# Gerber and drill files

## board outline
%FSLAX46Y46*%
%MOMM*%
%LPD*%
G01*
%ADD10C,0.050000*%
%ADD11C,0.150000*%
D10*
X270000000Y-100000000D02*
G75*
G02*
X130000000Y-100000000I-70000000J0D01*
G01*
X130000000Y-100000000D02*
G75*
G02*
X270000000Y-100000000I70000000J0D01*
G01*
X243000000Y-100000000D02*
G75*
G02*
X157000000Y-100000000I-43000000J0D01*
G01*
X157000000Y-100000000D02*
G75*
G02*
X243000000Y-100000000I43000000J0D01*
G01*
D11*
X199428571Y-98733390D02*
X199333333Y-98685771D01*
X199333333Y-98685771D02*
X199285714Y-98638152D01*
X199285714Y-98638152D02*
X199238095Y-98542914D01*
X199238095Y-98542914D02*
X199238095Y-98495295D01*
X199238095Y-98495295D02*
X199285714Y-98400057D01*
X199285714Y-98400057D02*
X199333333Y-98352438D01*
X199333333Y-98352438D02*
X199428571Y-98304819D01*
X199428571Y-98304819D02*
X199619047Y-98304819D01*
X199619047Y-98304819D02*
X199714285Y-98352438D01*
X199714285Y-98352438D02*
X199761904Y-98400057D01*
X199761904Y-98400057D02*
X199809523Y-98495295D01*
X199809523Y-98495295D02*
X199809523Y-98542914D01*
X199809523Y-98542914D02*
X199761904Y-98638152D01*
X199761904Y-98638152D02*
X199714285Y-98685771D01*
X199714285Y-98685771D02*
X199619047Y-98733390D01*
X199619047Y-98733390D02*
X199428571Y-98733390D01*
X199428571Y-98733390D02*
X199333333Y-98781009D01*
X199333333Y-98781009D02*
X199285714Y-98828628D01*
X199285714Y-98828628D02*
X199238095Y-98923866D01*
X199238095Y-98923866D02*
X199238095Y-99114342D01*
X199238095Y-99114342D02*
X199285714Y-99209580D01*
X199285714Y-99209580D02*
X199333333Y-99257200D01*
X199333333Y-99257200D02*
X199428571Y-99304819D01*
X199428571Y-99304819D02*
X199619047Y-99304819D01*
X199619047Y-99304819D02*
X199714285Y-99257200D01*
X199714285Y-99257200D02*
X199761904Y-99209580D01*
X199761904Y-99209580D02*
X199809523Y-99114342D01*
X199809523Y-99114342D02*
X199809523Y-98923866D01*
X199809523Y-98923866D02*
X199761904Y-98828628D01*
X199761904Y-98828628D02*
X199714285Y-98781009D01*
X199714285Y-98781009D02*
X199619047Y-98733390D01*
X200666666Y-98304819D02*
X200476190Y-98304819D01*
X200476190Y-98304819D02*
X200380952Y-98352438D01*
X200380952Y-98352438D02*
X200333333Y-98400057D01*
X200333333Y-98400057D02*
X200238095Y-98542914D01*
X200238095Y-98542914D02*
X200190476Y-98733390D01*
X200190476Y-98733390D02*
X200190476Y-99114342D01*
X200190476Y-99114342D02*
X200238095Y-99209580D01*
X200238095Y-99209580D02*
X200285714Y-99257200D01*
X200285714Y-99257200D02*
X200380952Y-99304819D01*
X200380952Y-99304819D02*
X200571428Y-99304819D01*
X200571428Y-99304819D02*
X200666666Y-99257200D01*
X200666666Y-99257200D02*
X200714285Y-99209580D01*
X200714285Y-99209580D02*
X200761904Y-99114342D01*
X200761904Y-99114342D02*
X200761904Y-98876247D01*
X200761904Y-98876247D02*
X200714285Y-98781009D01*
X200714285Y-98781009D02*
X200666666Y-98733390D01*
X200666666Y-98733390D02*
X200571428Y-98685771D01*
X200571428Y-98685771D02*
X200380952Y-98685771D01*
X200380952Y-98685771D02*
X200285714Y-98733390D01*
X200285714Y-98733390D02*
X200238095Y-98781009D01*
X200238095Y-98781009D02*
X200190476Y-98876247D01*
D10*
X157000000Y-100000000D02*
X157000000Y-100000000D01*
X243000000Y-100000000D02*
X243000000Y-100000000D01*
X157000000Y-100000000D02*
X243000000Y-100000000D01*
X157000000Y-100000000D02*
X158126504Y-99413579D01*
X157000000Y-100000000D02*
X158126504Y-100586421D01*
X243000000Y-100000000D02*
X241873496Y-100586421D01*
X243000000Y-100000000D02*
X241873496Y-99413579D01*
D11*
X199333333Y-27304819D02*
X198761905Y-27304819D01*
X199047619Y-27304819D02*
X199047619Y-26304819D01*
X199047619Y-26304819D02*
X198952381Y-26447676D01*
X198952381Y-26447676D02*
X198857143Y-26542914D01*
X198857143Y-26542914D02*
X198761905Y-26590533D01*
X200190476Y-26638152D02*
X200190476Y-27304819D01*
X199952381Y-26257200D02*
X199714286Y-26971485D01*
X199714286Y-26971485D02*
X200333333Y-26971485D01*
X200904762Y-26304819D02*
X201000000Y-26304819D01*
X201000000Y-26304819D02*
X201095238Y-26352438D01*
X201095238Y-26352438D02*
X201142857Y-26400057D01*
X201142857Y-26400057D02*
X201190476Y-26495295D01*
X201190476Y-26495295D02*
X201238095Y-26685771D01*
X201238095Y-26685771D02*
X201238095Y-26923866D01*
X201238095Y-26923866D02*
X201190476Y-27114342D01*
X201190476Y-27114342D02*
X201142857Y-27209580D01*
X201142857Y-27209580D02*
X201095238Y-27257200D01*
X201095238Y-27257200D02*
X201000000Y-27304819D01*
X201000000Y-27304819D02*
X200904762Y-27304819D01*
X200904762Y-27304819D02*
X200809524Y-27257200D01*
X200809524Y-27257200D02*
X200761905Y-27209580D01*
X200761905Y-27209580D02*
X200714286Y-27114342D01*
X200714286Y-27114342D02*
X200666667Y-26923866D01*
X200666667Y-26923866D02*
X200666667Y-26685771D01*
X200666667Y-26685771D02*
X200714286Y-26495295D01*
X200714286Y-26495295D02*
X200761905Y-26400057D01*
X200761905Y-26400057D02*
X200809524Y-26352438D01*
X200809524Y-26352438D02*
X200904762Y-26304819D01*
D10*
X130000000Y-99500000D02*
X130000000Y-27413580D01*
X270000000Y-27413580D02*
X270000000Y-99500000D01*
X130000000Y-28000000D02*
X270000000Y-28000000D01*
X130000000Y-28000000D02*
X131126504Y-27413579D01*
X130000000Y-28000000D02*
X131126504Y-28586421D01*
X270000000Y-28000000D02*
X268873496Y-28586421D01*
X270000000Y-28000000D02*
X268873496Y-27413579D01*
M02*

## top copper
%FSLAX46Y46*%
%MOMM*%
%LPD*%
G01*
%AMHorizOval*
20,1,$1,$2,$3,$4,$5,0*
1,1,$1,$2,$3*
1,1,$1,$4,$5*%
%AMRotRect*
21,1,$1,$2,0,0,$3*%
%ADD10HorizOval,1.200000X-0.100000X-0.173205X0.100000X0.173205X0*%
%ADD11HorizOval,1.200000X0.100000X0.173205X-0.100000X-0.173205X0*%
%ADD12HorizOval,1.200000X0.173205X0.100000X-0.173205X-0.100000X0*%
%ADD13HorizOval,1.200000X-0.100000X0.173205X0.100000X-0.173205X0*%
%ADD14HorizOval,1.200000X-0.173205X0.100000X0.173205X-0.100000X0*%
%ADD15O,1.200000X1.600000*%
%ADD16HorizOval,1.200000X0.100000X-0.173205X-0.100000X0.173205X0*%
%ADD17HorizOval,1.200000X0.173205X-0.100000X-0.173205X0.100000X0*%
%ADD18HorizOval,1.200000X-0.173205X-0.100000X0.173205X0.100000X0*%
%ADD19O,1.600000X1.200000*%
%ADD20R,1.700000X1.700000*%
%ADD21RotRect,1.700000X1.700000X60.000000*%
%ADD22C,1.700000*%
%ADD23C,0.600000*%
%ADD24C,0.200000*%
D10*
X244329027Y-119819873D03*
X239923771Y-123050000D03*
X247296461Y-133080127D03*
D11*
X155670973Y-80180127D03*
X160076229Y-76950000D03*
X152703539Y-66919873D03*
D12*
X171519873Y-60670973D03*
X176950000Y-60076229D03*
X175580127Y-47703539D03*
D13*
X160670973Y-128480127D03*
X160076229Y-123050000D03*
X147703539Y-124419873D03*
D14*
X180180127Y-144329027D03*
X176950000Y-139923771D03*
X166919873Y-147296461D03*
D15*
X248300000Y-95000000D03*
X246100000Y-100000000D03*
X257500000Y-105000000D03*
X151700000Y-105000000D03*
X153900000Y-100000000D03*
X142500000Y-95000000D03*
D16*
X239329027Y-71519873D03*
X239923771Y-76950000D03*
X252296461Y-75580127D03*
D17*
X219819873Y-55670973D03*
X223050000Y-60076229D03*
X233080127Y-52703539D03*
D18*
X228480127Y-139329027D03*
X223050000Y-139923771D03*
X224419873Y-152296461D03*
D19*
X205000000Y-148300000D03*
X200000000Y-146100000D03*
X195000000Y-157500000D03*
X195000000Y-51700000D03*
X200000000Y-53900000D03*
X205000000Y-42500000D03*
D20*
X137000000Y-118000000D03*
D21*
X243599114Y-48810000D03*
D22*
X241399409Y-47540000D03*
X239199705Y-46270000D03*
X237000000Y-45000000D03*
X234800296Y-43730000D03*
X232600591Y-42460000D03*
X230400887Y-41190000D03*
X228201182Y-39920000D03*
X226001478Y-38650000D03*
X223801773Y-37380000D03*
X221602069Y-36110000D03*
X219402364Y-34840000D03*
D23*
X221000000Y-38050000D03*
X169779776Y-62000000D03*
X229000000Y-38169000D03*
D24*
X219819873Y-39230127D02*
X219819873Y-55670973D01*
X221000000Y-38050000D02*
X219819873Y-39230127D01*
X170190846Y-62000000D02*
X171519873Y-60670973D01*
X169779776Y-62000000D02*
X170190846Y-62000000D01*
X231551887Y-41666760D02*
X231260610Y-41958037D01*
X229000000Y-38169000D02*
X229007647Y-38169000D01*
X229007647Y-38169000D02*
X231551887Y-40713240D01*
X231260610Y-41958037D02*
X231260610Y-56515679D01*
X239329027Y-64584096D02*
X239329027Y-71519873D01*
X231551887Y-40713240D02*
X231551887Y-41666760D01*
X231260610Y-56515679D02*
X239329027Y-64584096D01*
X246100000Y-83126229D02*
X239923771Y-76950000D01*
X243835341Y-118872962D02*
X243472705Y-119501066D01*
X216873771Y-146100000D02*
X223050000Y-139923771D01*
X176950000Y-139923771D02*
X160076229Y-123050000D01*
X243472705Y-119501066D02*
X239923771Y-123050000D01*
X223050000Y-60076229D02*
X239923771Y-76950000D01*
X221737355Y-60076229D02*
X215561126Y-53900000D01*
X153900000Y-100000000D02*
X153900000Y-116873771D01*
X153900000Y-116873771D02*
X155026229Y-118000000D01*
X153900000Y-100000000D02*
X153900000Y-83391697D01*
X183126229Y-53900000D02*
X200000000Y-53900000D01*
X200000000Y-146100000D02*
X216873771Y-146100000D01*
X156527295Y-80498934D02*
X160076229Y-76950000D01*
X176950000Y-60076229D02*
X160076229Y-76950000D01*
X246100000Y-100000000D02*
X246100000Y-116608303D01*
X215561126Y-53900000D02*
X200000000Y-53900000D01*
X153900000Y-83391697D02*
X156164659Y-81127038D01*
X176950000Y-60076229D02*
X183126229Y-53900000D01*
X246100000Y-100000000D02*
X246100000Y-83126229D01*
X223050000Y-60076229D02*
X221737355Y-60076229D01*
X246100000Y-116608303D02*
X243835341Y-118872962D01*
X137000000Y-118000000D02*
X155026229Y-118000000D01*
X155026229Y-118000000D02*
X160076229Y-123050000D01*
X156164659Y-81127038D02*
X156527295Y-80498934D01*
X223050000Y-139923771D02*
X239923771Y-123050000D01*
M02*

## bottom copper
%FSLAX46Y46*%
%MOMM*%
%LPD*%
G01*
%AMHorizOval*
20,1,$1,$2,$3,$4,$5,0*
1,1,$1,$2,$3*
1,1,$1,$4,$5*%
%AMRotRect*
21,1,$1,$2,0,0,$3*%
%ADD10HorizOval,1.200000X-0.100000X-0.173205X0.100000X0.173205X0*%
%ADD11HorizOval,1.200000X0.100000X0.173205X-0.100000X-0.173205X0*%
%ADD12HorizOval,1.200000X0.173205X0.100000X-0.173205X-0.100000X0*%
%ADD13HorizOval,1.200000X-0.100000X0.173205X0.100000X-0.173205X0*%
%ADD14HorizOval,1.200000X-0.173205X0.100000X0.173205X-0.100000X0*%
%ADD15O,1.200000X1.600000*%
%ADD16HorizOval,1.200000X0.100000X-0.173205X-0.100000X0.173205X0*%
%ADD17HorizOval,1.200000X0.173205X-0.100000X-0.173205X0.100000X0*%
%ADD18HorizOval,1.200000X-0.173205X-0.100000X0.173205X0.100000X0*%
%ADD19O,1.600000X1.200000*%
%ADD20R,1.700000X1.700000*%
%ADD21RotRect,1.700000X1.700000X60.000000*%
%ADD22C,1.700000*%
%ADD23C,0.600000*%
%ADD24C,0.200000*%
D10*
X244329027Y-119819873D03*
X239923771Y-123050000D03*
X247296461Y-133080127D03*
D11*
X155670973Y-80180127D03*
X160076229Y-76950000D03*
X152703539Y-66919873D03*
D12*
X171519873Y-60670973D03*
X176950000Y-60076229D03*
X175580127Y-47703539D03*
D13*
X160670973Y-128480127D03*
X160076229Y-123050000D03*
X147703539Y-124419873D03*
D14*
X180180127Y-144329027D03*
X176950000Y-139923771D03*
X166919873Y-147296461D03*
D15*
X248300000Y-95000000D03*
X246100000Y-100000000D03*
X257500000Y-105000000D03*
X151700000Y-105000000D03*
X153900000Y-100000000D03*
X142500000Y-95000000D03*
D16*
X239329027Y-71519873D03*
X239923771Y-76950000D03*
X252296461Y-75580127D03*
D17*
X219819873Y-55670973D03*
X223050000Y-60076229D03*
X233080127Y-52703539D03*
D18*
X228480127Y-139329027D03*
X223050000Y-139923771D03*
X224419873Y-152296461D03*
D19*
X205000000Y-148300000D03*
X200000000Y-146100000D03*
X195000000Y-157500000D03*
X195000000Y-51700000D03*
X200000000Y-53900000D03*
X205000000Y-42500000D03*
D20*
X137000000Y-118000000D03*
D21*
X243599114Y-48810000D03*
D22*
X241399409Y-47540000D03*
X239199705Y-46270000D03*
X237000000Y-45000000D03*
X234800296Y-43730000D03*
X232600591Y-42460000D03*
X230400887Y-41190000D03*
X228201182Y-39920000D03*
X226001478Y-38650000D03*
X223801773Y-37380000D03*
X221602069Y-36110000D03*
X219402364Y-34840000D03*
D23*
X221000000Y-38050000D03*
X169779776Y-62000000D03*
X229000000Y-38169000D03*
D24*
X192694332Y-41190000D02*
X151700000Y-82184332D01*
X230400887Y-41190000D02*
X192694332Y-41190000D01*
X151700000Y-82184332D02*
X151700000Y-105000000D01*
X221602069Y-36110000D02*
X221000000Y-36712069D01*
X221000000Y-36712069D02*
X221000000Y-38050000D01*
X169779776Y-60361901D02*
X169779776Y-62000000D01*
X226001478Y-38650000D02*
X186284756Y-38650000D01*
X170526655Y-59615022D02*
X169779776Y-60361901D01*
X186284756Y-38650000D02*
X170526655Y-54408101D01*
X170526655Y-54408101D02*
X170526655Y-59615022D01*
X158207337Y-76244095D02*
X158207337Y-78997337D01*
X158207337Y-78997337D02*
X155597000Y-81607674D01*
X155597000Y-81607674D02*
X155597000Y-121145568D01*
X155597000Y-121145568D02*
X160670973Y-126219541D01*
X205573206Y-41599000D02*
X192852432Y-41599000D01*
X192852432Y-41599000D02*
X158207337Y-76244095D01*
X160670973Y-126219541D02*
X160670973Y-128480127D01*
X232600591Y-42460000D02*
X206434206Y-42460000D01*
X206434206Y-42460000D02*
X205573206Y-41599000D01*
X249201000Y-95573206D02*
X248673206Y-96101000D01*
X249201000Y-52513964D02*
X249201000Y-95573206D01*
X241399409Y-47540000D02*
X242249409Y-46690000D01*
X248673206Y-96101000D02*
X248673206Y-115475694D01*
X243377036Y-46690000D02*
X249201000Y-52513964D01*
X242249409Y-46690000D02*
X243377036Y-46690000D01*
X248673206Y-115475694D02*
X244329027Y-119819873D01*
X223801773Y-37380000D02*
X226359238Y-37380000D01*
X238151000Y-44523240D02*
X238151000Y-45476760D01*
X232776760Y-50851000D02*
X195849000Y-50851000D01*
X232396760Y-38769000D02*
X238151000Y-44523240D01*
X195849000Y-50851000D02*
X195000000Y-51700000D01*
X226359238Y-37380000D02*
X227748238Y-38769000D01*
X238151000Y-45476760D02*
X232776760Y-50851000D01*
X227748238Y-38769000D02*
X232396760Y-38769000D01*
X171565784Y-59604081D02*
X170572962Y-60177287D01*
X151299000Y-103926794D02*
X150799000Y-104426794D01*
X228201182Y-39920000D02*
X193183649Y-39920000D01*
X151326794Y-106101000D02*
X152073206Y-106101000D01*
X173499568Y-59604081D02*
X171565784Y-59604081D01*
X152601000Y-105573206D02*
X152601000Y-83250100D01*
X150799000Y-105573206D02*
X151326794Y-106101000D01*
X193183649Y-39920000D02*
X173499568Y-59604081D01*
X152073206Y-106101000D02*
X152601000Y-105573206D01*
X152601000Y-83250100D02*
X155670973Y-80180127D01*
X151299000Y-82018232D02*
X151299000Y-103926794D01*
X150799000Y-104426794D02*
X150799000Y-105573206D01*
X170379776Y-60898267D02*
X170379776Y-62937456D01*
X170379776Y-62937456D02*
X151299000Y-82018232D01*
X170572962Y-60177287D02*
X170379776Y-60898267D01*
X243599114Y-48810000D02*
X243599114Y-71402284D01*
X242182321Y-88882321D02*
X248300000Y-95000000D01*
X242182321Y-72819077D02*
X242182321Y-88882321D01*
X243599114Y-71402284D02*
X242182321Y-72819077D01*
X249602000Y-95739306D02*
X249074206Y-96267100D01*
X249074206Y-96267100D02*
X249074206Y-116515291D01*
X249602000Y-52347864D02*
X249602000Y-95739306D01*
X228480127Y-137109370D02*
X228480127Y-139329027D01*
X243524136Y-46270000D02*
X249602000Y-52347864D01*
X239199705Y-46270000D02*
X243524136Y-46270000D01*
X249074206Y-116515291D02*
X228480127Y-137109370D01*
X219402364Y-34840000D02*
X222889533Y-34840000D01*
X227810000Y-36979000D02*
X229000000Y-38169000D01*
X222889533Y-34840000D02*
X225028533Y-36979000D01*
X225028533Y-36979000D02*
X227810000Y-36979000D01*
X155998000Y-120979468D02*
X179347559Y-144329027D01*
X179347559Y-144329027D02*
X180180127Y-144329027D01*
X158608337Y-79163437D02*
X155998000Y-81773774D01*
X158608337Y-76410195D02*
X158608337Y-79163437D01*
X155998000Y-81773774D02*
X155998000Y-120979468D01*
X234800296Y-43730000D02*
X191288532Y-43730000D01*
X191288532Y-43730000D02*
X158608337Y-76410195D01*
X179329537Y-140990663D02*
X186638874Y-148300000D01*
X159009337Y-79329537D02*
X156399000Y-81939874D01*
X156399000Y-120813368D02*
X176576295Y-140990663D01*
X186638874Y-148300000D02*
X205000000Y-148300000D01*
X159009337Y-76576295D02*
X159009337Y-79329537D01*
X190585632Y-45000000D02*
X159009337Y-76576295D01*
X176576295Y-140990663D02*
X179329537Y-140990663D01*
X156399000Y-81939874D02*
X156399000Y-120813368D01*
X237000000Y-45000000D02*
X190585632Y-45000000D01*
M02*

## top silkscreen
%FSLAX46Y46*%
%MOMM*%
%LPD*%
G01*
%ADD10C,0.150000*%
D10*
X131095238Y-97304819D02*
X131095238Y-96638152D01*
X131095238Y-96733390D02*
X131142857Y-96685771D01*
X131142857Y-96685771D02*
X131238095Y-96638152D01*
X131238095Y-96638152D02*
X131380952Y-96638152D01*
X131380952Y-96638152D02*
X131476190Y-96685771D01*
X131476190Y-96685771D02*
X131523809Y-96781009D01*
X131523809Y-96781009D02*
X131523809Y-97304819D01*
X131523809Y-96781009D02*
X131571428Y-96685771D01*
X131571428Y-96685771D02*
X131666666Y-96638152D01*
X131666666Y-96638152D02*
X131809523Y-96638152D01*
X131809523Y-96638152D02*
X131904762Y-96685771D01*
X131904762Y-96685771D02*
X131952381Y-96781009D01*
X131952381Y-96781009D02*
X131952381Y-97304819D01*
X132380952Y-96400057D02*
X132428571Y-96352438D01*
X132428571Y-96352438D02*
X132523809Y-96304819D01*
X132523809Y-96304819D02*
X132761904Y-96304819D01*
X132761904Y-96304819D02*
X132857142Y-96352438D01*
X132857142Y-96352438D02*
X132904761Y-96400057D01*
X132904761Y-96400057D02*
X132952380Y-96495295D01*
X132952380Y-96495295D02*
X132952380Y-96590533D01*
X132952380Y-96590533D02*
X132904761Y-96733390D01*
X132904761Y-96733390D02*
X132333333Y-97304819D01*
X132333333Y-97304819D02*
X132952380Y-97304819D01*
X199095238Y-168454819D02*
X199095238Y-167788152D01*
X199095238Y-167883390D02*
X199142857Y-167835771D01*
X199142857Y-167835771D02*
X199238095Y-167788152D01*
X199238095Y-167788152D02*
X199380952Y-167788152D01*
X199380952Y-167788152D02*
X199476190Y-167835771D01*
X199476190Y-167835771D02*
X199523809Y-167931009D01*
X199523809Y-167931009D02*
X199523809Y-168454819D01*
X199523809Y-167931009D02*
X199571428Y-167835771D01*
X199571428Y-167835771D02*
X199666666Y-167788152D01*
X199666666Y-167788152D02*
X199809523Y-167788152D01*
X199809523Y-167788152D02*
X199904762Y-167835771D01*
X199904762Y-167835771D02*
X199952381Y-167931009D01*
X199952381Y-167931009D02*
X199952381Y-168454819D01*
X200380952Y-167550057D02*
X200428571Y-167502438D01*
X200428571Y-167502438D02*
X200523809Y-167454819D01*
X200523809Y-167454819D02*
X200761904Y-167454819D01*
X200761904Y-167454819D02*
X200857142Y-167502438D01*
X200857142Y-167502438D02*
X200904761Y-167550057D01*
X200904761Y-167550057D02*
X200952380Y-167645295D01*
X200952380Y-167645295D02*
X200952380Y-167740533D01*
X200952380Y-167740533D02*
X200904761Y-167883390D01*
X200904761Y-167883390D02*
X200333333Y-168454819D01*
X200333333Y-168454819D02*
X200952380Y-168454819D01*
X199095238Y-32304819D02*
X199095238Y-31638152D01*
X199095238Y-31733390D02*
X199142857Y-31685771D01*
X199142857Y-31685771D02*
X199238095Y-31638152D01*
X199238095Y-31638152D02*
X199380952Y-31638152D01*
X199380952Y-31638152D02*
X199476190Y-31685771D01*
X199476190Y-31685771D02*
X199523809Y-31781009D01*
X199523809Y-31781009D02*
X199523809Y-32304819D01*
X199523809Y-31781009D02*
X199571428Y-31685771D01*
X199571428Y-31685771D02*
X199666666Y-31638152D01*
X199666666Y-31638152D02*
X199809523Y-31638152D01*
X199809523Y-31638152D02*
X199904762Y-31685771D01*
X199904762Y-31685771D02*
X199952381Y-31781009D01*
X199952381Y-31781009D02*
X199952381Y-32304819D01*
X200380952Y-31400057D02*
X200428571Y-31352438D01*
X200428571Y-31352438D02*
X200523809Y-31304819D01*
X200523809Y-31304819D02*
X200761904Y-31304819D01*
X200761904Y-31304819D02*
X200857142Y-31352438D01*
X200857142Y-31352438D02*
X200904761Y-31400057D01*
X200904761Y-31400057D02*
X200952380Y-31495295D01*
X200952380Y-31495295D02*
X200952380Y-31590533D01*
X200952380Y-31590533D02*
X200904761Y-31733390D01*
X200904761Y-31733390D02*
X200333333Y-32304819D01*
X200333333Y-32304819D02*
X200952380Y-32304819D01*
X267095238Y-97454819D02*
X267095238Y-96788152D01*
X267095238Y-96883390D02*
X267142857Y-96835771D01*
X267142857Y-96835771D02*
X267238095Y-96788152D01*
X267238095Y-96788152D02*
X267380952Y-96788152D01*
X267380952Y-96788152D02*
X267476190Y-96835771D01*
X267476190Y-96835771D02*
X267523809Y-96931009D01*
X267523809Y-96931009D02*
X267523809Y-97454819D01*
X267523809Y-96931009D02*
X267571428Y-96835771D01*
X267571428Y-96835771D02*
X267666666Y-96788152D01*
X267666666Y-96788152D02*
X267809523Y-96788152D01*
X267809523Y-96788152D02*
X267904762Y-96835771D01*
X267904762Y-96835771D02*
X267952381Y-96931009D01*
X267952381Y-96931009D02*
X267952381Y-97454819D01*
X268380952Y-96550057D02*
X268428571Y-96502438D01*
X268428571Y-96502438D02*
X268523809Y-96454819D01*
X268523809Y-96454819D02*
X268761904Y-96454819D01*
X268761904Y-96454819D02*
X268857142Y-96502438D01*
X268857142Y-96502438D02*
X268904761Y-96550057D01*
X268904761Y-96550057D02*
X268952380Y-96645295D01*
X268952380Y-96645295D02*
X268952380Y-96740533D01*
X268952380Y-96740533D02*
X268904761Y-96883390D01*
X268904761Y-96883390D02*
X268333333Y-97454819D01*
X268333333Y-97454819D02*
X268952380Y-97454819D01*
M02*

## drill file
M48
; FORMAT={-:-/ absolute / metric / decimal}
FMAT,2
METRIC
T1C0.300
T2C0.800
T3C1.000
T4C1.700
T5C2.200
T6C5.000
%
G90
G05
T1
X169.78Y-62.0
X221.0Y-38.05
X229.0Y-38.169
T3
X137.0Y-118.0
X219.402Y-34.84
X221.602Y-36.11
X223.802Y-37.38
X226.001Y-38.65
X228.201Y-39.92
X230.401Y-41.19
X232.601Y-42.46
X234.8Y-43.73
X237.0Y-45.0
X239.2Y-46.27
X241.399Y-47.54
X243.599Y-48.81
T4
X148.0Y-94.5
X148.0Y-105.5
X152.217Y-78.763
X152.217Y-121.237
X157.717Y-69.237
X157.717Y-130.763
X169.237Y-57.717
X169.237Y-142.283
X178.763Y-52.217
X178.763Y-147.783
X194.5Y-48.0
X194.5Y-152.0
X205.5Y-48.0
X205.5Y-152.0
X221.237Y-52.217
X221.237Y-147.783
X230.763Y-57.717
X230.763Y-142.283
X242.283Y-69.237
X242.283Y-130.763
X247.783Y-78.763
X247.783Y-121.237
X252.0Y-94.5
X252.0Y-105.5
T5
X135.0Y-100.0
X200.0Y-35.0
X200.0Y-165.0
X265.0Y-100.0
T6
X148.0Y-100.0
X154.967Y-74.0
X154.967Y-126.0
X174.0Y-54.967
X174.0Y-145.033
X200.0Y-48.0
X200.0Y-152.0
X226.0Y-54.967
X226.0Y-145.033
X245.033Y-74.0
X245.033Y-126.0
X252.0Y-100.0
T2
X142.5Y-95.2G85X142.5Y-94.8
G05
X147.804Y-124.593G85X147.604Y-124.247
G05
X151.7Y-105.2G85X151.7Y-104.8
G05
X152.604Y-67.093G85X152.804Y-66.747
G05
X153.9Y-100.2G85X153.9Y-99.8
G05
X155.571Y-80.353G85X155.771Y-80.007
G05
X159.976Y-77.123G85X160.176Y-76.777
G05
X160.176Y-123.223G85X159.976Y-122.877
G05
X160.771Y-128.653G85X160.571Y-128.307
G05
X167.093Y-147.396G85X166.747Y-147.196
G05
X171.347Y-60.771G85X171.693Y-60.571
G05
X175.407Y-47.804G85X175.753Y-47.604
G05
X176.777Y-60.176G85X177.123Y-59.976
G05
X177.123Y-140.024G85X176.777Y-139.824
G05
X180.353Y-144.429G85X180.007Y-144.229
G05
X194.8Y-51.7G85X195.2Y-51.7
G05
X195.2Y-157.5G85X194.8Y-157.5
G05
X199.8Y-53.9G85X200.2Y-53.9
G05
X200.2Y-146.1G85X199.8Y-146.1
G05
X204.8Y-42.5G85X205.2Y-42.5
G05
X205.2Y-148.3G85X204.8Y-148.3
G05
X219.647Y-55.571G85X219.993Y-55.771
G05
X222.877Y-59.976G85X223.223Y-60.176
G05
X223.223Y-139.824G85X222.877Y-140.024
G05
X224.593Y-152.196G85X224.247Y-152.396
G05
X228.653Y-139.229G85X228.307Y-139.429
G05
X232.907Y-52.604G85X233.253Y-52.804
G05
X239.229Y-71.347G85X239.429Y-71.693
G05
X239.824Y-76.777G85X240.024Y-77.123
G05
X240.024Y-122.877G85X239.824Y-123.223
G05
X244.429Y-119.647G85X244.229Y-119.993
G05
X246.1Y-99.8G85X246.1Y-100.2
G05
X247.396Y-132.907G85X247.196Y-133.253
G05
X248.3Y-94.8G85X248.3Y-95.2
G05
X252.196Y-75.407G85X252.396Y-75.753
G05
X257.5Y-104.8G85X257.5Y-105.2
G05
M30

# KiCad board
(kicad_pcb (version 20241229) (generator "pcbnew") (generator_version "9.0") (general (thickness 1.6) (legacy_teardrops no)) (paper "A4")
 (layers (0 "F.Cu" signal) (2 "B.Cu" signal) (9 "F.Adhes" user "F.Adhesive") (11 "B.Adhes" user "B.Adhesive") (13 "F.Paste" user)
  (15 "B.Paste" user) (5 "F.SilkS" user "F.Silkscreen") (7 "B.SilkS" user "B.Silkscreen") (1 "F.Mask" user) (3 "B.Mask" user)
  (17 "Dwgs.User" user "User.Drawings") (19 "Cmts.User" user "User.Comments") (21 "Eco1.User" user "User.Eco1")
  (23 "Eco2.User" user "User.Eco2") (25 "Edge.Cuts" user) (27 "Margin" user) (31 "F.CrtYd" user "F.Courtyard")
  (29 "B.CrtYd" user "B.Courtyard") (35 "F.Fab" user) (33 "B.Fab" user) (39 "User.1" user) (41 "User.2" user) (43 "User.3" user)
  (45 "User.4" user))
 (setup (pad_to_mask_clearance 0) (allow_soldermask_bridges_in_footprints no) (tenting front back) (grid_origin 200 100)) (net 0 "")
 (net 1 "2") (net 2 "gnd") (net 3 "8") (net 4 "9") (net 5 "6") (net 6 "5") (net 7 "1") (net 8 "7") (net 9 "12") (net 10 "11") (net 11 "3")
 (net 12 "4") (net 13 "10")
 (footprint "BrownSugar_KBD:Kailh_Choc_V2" (layer "F.Cu") (at 245.033321 126 -120)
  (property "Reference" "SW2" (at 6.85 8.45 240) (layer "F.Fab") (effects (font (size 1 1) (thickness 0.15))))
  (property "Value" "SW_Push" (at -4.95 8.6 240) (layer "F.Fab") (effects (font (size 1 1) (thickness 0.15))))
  (pad "" np_thru_hole circle (at -5.5 0 240) (size 1.7 1.7) (drill 1.7) (layers "*.Cu" "*.Mask"))
  (pad "" np_thru_hole circle (at 0 0 240) (size 5 5) (drill 5) (layers "*.Cu" "*.Mask"))
  (pad "" np_thru_hole circle (at 5.5 0 240) (size 1.7 1.7) (drill 1.7) (layers "*.Cu" "*.Mask"))
  (pad "1" thru_hole oval (at -5 3.7 240) (size 1.6 1.2) (drill oval 1.2 0.8) (layers "*.Cu" "*.Mask") (remove_unused_layers no) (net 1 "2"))
  (pad "2" thru_hole oval (at 0 5.9 240) (size 1.6 1.2) (drill oval 1.2 0.8) (layers "*.Cu" "*.Mask") (remove_unused_layers no)
   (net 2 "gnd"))
  (pad "MP" thru_hole oval (at 5 -5.5 240) (size 1.6 1.2) (drill oval 1.2 0.8) (layers "*.Cu" "*.Mask") (remove_unused_layers no)))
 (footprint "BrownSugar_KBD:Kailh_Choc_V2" (layer "F.Cu") (at 154.966679 74 60)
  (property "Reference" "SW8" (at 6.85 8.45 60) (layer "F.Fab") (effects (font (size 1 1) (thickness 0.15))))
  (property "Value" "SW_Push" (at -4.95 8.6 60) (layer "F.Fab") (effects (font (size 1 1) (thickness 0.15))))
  (pad "" np_thru_hole circle (at -5.5 0 60) (size 1.7 1.7) (drill 1.7) (layers "*.Cu" "*.Mask"))
  (pad "" np_thru_hole circle (at 0 0 60) (size 5 5) (drill 5) (layers "*.Cu" "*.Mask"))
  (pad "" np_thru_hole circle (at 5.5 0 60) (size 1.7 1.7) (drill 1.7) (layers "*.Cu" "*.Mask"))
  (pad "1" thru_hole oval (at -5 3.7 60) (size 1.6 1.2) (drill oval 1.2 0.8) (layers "*.Cu" "*.Mask") (remove_unused_layers no) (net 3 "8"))
  (pad "2" thru_hole oval (at 0 5.9 60) (size 1.6 1.2) (drill oval 1.2 0.8) (layers "*.Cu" "*.Mask") (remove_unused_layers no) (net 2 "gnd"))
  (pad "MP" thru_hole oval (at 5 -5.5 60) (size 1.6 1.2) (drill oval 1.2 0.8) (layers "*.Cu" "*.Mask") (remove_unused_layers no)))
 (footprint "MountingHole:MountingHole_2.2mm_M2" (layer "F.Cu") (at 135 100)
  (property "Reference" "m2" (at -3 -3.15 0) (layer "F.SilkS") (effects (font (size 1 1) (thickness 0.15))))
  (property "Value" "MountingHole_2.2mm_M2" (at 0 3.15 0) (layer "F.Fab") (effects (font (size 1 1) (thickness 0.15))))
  (pad "" np_thru_hole circle (at 0 0) (size 2.2 2.2) (drill 2.2) (layers "*.Cu" "*.Mask")))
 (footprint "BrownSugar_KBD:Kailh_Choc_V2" (layer "F.Cu") (at 174 54.966679 30)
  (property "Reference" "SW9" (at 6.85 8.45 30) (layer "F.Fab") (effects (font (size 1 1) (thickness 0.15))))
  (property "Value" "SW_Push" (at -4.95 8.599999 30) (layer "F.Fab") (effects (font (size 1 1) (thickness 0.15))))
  (pad "" np_thru_hole circle (at -5.5 0 30) (size 1.7 1.7) (drill 1.7) (layers "*.Cu" "*.Mask"))
  (pad "" np_thru_hole circle (at 0 0 30) (size 5 5) (drill 5) (layers "*.Cu" "*.Mask"))
  (pad "" np_thru_hole circle (at 5.5 0 30) (size 1.7 1.7) (drill 1.7) (layers "*.Cu" "*.Mask"))
  (pad "1" thru_hole oval (at -5 3.7 30) (size 1.6 1.2) (drill oval 1.2 0.8) (layers "*.Cu" "*.Mask") (remove_unused_layers no) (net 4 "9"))
  (pad "2" thru_hole oval (at 0 5.9 30) (size 1.6 1.2) (drill oval 1.2 0.8) (layers "*.Cu" "*.Mask") (remove_unused_layers no) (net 2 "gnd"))
  (pad "MP" thru_hole oval (at 5 -5.5 30) (size 1.6 1.2) (drill oval 1.2 0.8) (layers "*.Cu" "*.Mask") (remove_unused_layers no)))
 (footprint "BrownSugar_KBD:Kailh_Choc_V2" (layer "F.Cu") (at 154.966679 126 120)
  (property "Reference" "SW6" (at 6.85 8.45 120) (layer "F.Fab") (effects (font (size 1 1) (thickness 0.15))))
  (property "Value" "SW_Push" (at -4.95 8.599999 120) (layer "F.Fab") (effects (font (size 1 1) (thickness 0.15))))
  (pad "" np_thru_hole circle (at -5.5 0 120) (size 1.7 1.7) (drill 1.7) (layers "*.Cu" "*.Mask"))
  (pad "" np_thru_hole circle (at 0 0 120) (size 5 5) (drill 5) (layers "*.Cu" "*.Mask"))
  (pad "" np_thru_hole circle (at 5.5 0 120) (size 1.7 1.7) (drill 1.7) (layers "*.Cu" "*.Mask"))
  (pad "1" thru_hole oval (at -5 3.7 120) (size 1.6 1.2) (drill oval 1.2 0.8) (layers "*.Cu" "*.Mask") (remove_unused_layers no) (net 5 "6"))
  (pad "2" thru_hole oval (at 0 5.9 120) (size 1.6 1.2) (drill oval 1.2 0.8) (layers "*.Cu" "*.Mask") (remove_unused_layers no)
   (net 2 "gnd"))
  (pad "MP" thru_hole oval (at 5 -5.5 120) (size 1.6 1.2) (drill oval 1.2 0.8) (layers "*.Cu" "*.Mask") (remove_unused_layers no)))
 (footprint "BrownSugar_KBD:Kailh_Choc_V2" (layer "F.Cu") (at 174 145.033321 150)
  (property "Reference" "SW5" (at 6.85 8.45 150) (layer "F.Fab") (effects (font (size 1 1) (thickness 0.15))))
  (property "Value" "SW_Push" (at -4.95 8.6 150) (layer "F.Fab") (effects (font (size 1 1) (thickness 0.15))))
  (pad "" np_thru_hole circle (at -5.5 0 150) (size 1.7 1.7) (drill 1.7) (layers "*.Cu" "*.Mask"))
  (pad "" np_thru_hole circle (at 0 0 150) (size 5 5) (drill 5) (layers "*.Cu" "*.Mask"))
  (pad "" np_thru_hole circle (at 5.5 0 150) (size 1.7 1.7) (drill 1.7) (layers "*.Cu" "*.Mask"))
  (pad "1" thru_hole oval (at -5 3.7 150) (size 1.6 1.2) (drill oval 1.2 0.8) (layers "*.Cu" "*.Mask") (remove_unused_layers no) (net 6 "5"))
  (pad "2" thru_hole oval (at 0 5.9 150) (size 1.6 1.2) (drill oval 1.2 0.8) (layers "*.Cu" "*.Mask") (remove_unused_layers no)
   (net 2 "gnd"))
  (pad "MP" thru_hole oval (at 5 -5.5 150) (size 1.6 1.2) (drill oval 1.2 0.8) (layers "*.Cu" "*.Mask") (remove_unused_layers no)))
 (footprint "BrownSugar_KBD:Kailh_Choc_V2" (layer "F.Cu") (at 252 100 -90)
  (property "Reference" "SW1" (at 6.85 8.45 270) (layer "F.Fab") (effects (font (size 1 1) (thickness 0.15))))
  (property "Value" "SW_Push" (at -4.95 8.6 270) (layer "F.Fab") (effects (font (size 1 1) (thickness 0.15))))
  (pad "" np_thru_hole circle (at -5.5 0 270) (size 1.7 1.7) (drill 1.7) (layers "*.Cu" "*.Mask"))
  (pad "" np_thru_hole circle (at 0 0 270) (size 5 5) (drill 5) (layers "*.Cu" "*.Mask"))
  (pad "" np_thru_hole circle (at 5.5 0 270) (size 1.7 1.7) (drill 1.7) (layers "*.Cu" "*.Mask"))
  (pad "1" thru_hole oval (at -5 3.7 270) (size 1.6 1.2) (drill oval 1.2 0.8) (layers "*.Cu" "*.Mask") (remove_unused_layers no) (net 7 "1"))
  (pad "2" thru_hole oval (at 0 5.9 270) (size 1.6 1.2) (drill oval 1.2 0.8) (layers "*.Cu" "*.Mask") (remove_unused_layers no)
   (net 2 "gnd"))
  (pad "MP" thru_hole oval (at 5 -5.5 270) (size 1.6 1.2) (drill oval 1.2 0.8) (layers "*.Cu" "*.Mask") (remove_unused_layers no)))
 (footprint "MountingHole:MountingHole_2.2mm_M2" (layer "F.Cu") (at 200 165)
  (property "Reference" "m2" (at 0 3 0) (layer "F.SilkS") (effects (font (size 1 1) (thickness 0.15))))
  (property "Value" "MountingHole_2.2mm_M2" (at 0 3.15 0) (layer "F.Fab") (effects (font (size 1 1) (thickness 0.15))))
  (pad "" np_thru_hole circle (at 0 0) (size 2.2 2.2) (drill 2.2) (layers "*.Cu" "*.Mask")))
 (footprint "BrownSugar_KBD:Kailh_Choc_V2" (layer "F.Cu") (at 148 100 90)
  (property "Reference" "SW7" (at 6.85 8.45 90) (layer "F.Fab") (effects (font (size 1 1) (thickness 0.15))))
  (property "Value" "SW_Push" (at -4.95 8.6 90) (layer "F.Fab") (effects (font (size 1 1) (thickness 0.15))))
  (pad "" np_thru_hole circle (at -5.5 0 90) (size 1.7 1.7) (drill 1.7) (layers "*.Cu" "*.Mask"))
  (pad "" np_thru_hole circle (at 0 0 90) (size 5 5) (drill 5) (layers "*.Cu" "*.Mask"))
  (pad "" np_thru_hole circle (at 5.5 0 90) (size 1.7 1.7) (drill 1.7) (layers "*.Cu" "*.Mask"))
  (pad "1" thru_hole oval (at -5 3.7 90) (size 1.6 1.2) (drill oval 1.2 0.8) (layers "*.Cu" "*.Mask") (remove_unused_layers no) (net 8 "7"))
  (pad "2" thru_hole oval (at 0 5.9 90) (size 1.6 1.2) (drill oval 1.2 0.8) (layers "*.Cu" "*.Mask") (remove_unused_layers no) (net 2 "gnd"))
  (pad "MP" thru_hole oval (at 5 -5.5 90) (size 1.6 1.2) (drill oval 1.2 0.8) (layers "*.Cu" "*.Mask") (remove_unused_layers no)))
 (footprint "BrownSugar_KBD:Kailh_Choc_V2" (layer "F.Cu") (at 245.033321 74 -60)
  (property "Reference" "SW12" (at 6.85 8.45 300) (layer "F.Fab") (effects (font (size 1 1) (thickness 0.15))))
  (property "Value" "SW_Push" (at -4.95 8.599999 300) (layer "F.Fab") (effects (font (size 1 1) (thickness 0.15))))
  (pad "" np_thru_hole circle (at -5.5 0 300) (size 1.7 1.7) (drill 1.7) (layers "*.Cu" "*.Mask"))
  (pad "" np_thru_hole circle (at 0 0 300) (size 5 5) (drill 5) (layers "*.Cu" "*.Mask"))
  (pad "" np_thru_hole circle (at 5.5 0 300) (size 1.7 1.7) (drill 1.7) (layers "*.Cu" "*.Mask"))
  (pad "1" thru_hole oval (at -5 3.7 300) (size 1.6 1.2) (drill oval 1.2 0.8) (layers "*.Cu" "*.Mask") (remove_unused_layers no)
   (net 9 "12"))
  (pad "2" thru_hole oval (at 0 5.9 300) (size 1.6 1.2) (drill oval 1.2 0.8) (layers "*.Cu" "*.Mask") (remove_unused_layers no)
   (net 2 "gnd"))
  (pad "MP" thru_hole oval (at 5 -5.5 300) (size 1.6 1.2) (drill oval 1.2 0.8) (layers "*.Cu" "*.Mask") (remove_unused_layers no)))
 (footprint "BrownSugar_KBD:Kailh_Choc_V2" (layer "F.Cu") (at 226 54.966679 -30)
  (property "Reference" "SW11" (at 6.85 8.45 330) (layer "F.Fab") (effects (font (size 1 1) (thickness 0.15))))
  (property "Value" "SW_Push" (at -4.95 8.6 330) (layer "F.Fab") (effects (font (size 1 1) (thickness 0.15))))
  (pad "" np_thru_hole circle (at -5.5 0 330) (size 1.7 1.7) (drill 1.7) (layers "*.Cu" "*.Mask"))
  (pad "" np_thru_hole circle (at 0 0 330) (size 5 5) (drill 5) (layers "*.Cu" "*.Mask"))
  (pad "" np_thru_hole circle (at 5.5 0 330) (size 1.7 1.7) (drill 1.7) (layers "*.Cu" "*.Mask"))
  (pad "1" thru_hole oval (at -5 3.7 330) (size 1.6 1.2) (drill oval 1.2 0.8) (layers "*.Cu" "*.Mask") (remove_unused_layers no)
   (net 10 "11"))
  (pad "2" thru_hole oval (at 0 5.9 330) (size 1.6 1.2) (drill oval 1.2 0.8) (layers "*.Cu" "*.Mask") (remove_unused_layers no)
   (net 2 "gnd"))
  (pad "MP" thru_hole oval (at 5 -5.5 330) (size 1.6 1.2) (drill oval 1.2 0.8) (layers "*.Cu" "*.Mask") (remove_unused_layers no)))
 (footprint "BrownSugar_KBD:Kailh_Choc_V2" (layer "F.Cu") (at 226 145.033321 -150)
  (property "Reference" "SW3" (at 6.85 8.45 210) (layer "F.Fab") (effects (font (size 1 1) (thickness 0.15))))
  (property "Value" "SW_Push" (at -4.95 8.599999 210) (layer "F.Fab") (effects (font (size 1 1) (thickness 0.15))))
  (pad "" np_thru_hole circle (at -5.5 0 210) (size 1.7 1.7) (drill 1.7) (layers "*.Cu" "*.Mask"))
  (pad "" np_thru_hole circle (at 0 0 210) (size 5 5) (drill 5) (layers "*.Cu" "*.Mask"))
  (pad "" np_thru_hole circle (at 5.5 0 210) (size 1.7 1.7) (drill 1.7) (layers "*.Cu" "*.Mask"))
  (pad "1" thru_hole oval (at -5 3.7 210) (size 1.6 1.2) (drill oval 1.2 0.8) (layers "*.Cu" "*.Mask") (remove_unused_layers no)
   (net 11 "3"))
  (pad "2" thru_hole oval (at 0 5.9 210) (size 1.6 1.2) (drill oval 1.2 0.8) (layers "*.Cu" "*.Mask") (remove_unused_layers no)
   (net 2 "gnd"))
  (pad "MP" thru_hole oval (at 5 -5.5 210) (size 1.6 1.2) (drill oval 1.2 0.8) (layers "*.Cu" "*.Mask") (remove_unused_layers no)))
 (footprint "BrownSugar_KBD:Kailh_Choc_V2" (layer "F.Cu") (at 200 152 180)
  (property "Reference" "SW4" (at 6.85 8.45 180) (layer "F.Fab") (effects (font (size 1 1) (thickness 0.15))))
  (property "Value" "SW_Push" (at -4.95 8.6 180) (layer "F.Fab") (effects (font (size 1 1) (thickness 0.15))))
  (pad "" np_thru_hole circle (at -5.5 0 180) (size 1.7 1.7) (drill 1.7) (layers "*.Cu" "*.Mask"))
  (pad "" np_thru_hole circle (at 0 0 180) (size 5 5) (drill 5) (layers "*.Cu" "*.Mask"))
  (pad "" np_thru_hole circle (at 5.5 0 180) (size 1.7 1.7) (drill 1.7) (layers "*.Cu" "*.Mask"))
  (pad "1" thru_hole oval (at -5 3.7 180) (size 1.6 1.2) (drill oval 1.2 0.8) (layers "*.Cu" "*.Mask") (remove_unused_layers no)
   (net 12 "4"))
  (pad "2" thru_hole oval (at 0 5.9 180) (size 1.6 1.2) (drill oval 1.2 0.8) (layers "*.Cu" "*.Mask") (remove_unused_layers no)
   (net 2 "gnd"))
  (pad "MP" thru_hole oval (at 5 -5.5 180) (size 1.6 1.2) (drill oval 1.2 0.8) (layers "*.Cu" "*.Mask") (remove_unused_layers no)))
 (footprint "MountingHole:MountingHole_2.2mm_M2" (layer "F.Cu") (at 200 35)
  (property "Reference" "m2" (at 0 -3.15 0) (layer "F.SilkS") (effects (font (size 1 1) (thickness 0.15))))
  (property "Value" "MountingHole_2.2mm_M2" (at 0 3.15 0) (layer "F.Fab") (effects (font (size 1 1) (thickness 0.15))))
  (pad "" np_thru_hole circle (at 0 0) (size 2.2 2.2) (drill 2.2) (layers "*.Cu" "*.Mask")))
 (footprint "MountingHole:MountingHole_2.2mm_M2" (layer "F.Cu") (at 265 100)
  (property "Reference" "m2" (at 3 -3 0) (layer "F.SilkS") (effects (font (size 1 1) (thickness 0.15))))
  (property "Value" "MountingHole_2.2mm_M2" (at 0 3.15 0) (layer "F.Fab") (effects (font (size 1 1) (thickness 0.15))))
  (pad "" np_thru_hole circle (at 0 0) (size 2.2 2.2) (drill 2.2) (layers "*.Cu" "*.Mask")))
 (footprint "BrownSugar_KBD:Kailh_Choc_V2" (layer "F.Cu") (at 200 48)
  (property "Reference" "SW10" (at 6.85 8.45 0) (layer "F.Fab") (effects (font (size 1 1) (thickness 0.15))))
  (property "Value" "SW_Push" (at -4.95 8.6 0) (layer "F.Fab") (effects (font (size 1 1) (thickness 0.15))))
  (pad "" np_thru_hole circle (at -5.5 0) (size 1.7 1.7) (drill 1.7) (layers "*.Cu" "*.Mask"))
  (pad "" np_thru_hole circle (at 0 0) (size 5 5) (drill 5) (layers "*.Cu" "*.Mask"))
  (pad "" np_thru_hole circle (at 5.5 0) (size 1.7 1.7) (drill 1.7) (layers "*.Cu" "*.Mask"))
  (pad "1" thru_hole oval (at -5 3.7) (size 1.6 1.2) (drill oval 1.2 0.8) (layers "*.Cu" "*.Mask") (remove_unused_layers no) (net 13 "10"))
  (pad "2" thru_hole oval (at 0 5.9) (size 1.6 1.2) (drill oval 1.2 0.8) (layers "*.Cu" "*.Mask") (remove_unused_layers no) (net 2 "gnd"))
  (pad "MP" thru_hole oval (at 5 -5.5) (size 1.6 1.2) (drill oval 1.2 0.8) (layers "*.Cu" "*.Mask") (remove_unused_layers no)))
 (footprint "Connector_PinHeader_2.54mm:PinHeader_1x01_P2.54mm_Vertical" (layer "B.Cu") (at 137 118 180)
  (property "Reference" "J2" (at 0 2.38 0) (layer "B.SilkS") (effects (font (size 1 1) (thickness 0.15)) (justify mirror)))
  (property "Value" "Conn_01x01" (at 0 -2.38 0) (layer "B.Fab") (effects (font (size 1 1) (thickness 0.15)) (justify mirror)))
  (pad "1" thru_hole rect (at 0 0 180) (size 1.7 1.7) (drill 1) (layers "*.Cu" "*.Mask") (remove_unused_layers no) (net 2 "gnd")))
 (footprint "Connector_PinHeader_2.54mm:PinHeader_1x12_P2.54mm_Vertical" (layer "B.Cu") (at 243.599114 48.81 60)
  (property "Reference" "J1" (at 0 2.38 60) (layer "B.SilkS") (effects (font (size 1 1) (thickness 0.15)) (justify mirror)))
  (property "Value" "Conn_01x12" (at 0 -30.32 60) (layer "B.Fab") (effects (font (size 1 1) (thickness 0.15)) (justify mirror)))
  (pad "1" thru_hole rect (at 0 0 60) (size 1.7 1.7) (drill 1) (layers "*.Cu" "*.Mask") (remove_unused_layers no) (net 7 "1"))
  (pad "2" thru_hole circle (at 0 -2.54 60) (size 1.7 1.7) (drill 1) (layers "*.Cu" "*.Mask") (remove_unused_layers no) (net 1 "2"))
  (pad "3" thru_hole circle (at 0 -5.08 60) (size 1.7 1.7) (drill 1) (layers "*.Cu" "*.Mask") (remove_unused_layers no) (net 11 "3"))
  (pad "4" thru_hole circle (at 0 -7.62 60) (size 1.7 1.7) (drill 1) (layers "*.Cu" "*.Mask") (remove_unused_layers no) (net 12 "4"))
  (pad "5" thru_hole circle (at 0 -10.16 60) (size 1.7 1.7) (drill 1) (layers "*.Cu" "*.Mask") (remove_unused_layers no) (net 6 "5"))
  (pad "6" thru_hole circle (at 0 -12.7 60) (size 1.7 1.7) (drill 1) (layers "*.Cu" "*.Mask") (remove_unused_layers no) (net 5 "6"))
  (pad "7" thru_hole circle (at 0 -15.24 60) (size 1.7 1.7) (drill 1) (layers "*.Cu" "*.Mask") (remove_unused_layers no) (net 8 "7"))
  (pad "8" thru_hole circle (at 0 -17.78 60) (size 1.7 1.7) (drill 1) (layers "*.Cu" "*.Mask") (remove_unused_layers no) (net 3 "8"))
  (pad "9" thru_hole circle (at 0 -20.32 60) (size 1.7 1.7) (drill 1) (layers "*.Cu" "*.Mask") (remove_unused_layers no) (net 4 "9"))
  (pad "10" thru_hole circle (at 0 -22.86 60) (size 1.7 1.7) (drill 1) (layers "*.Cu" "*.Mask") (remove_unused_layers no) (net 13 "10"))
  (pad "11" thru_hole circle (at 0 -25.4 60) (size 1.7 1.7) (drill 1) (layers "*.Cu" "*.Mask") (remove_unused_layers no) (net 10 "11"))
  (pad "12" thru_hole circle (at 0 -27.94 60) (size 1.7 1.7) (drill 1) (layers "*.Cu" "*.Mask") (remove_unused_layers no) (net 9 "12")))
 (gr_circle (center 200 100) (end 270 100) (stroke (width 0.05) (type default)) (fill no) (layer "Edge.Cuts"))
 (gr_circle (center 200 100) (end 243 100) (stroke (width 0.05) (type default)) (fill no) (layer "Edge.Cuts"))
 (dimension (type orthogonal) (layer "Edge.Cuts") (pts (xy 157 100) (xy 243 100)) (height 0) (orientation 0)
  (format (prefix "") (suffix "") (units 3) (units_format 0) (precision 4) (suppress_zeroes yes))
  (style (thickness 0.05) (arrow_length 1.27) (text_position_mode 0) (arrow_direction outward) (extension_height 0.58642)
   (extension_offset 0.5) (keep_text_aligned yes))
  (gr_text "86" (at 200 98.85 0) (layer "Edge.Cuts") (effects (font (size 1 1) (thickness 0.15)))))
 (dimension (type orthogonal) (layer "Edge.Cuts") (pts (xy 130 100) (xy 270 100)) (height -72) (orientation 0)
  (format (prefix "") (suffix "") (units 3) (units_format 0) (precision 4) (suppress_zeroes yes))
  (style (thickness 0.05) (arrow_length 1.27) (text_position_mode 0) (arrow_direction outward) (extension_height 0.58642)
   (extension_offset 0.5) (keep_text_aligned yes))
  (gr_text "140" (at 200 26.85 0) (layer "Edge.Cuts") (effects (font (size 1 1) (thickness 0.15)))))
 (segment (start 192.694332 41.19) (end 151.7 82.184332) (width 0.2) (layer "B.Cu") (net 8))
 (segment (start 230.400887 41.19) (end 192.694332 41.19) (width 0.2) (layer "B.Cu") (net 8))
 (segment (start 151.7 82.184332) (end 151.7 105) (width 0.2) (layer "B.Cu") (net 8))
 (segment (start 219.819873 39.230127) (end 219.819873 55.670973) (width 0.2) (layer "F.Cu") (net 10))
 (segment (start 221 38.05) (end 219.819873 39.230127) (width 0.2) (layer "F.Cu") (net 10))
 (via (at 221 38.05) (size 0.6) (drill 0.3) (layers "F.Cu" "B.Cu") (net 10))
 (segment (start 221.602069 36.11) (end 221 36.712069) (width 0.2) (layer "B.Cu") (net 10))
 (segment (start 221 36.712069) (end 221 38.05) (width 0.2) (layer "B.Cu") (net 10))
 (segment (start 170.190846 62) (end 171.519873 60.670973) (width 0.2) (layer "F.Cu") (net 4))
 (segment (start 169.779776 62) (end 170.190846 62) (width 0.2) (layer "F.Cu") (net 4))
 (via (at 169.779776 62) (size 0.6) (drill 0.3) (layers "F.Cu" "B.Cu") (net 4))
 (segment (start 169.779776 60.361901) (end 169.779776 62) (width 0.2) (layer "B.Cu") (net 4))
 (segment (start 226.001478 38.65) (end 186.284756 38.65) (width 0.2) (layer "B.Cu") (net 4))
 (segment (start 170.526655 59.615022) (end 169.779776 60.361901) (width 0.2) (layer "B.Cu") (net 4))
 (segment (start 186.284756 38.65) (end 170.526655 54.408101) (width 0.2) (layer "B.Cu") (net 4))
 (segment (start 170.526655 54.408101) (end 170.526655 59.615022) (width 0.2) (layer "B.Cu") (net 4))
 (segment (start 158.207337 76.244095) (end 158.207337 78.997337) (width 0.2) (layer "B.Cu") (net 5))
 (segment (start 158.207337 78.997337) (end 155.597 81.607674) (width 0.2) (layer "B.Cu") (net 5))
 (segment (start 155.597 81.607674) (end 155.597 121.145568) (width 0.2) (layer "B.Cu") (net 5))
 (segment (start 155.597 121.145568) (end 160.670973 126.219541) (width 0.2) (layer "B.Cu") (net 5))
 (segment (start 205.573206 41.599) (end 192.852432 41.599) (width 0.2) (layer "B.Cu") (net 5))
 (segment (start 192.852432 41.599) (end 158.207337 76.244095) (width 0.2) (layer "B.Cu") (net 5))
 (segment (start 160.670973 126.219541) (end 160.670973 128.480127) (width 0.2) (layer "B.Cu") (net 5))
 (segment (start 232.600591 42.46) (end 206.434206 42.46) (width 0.2) (layer "B.Cu") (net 5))
 (segment (start 206.434206 42.46) (end 205.573206 41.599) (width 0.2) (layer "B.Cu") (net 5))
 (segment (start 249.201 95.573206) (end 248.673206 96.101) (width 0.2) (layer "B.Cu") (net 1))
 (segment (start 249.201 52.513964) (end 249.201 95.573206) (width 0.2) (layer "B.Cu") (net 1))
 (segment (start 241.399409 47.54) (end 242.249409 46.69) (width 0.2) (layer "B.Cu") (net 1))
 (segment (start 248.673206 96.101) (end 248.673206 115.475694) (width 0.2) (layer "B.Cu") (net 1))
 (segment (start 243.377036 46.69) (end 249.201 52.513964) (width 0.2) (layer "B.Cu") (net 1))
 (segment (start 242.249409 46.69) (end 243.377036 46.69) (width 0.2) (layer "B.Cu") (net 1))
 (segment (start 248.673206 115.475694) (end 244.329027 119.819873) (width 0.2) (layer "B.Cu") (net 1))
 (segment (start 223.801773 37.38) (end 226.359238 37.38) (width 0.2) (layer "B.Cu") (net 13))
 (segment (start 238.151 44.52324) (end 238.151 45.47676) (width 0.2) (layer "B.Cu") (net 13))
 (segment (start 232.77676 50.851) (end 195.849 50.851) (width 0.2) (layer "B.Cu") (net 13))
 (segment (start 232.39676 38.769) (end 238.151 44.52324) (width 0.2) (layer "B.Cu") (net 13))
 (segment (start 195.849 50.851) (end 195 51.7) (width 0.2) (layer "B.Cu") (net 13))
 (segment (start 226.359238 37.38) (end 227.748238 38.769) (width 0.2) (layer "B.Cu") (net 13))
 (segment (start 238.151 45.47676) (end 232.77676 50.851) (width 0.2) (layer "B.Cu") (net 13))
 (segment (start 227.748238 38.769) (end 232.39676 38.769) (width 0.2) (layer "B.Cu") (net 13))
 (segment (start 171.565784 59.604081) (end 170.572962 60.177287) (width 0.2) (layer "B.Cu") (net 3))
 (segment (start 151.299 103.926794) (end 150.799 104.426794) (width 0.2) (layer "B.Cu") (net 3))
 (segment (start 228.201182 39.92) (end 193.183649 39.92) (width 0.2) (layer "B.Cu") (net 3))
 (segment (start 151.326794 106.101) (end 152.073206 106.101) (width 0.2) (layer "B.Cu") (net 3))
 (segment (start 173.499568 59.604081) (end 171.565784 59.604081) (width 0.2) (layer "B.Cu") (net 3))
 (segment (start 152.601 105.573206) (end 152.601 83.2501) (width 0.2) (layer "B.Cu") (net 3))
 (segment (start 150.799 105.573206) (end 151.326794 106.101) (width 0.2) (layer "B.Cu") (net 3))
 (segment (start 193.183649 39.92) (end 173.499568 59.604081) (width 0.2) (layer "B.Cu") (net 3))
 (segment (start 152.073206 106.101) (end 152.601 105.573206) (width 0.2) (layer "B.Cu") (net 3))
 (segment (start 152.601 83.2501) (end 155.670973 80.180127) (width 0.2) (layer "B.Cu") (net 3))
 (segment (start 151.299 82.018232) (end 151.299 103.926794) (width 0.2) (layer "B.Cu") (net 3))
 (segment (start 150.799 104.426794) (end 150.799 105.573206) (width 0.2) (layer "B.Cu") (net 3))
 (segment (start 170.379776 60.898267) (end 170.379776 62.937456) (width 0.2) (layer "B.Cu") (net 3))
 (segment (start 170.379776 62.937456) (end 151.299 82.018232) (width 0.2) (layer "B.Cu") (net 3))
 (segment (start 170.572962 60.177287) (end 170.379776 60.898267) (width 0.2) (layer "B.Cu") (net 3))
 (segment (start 243.599114 48.81) (end 243.599114 71.402284) (width 0.2) (layer "B.Cu") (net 7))
 (segment (start 242.182321 88.882321) (end 248.3 95) (width 0.2) (layer "B.Cu") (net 7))
 (segment (start 242.182321 72.819077) (end 242.182321 88.882321) (width 0.2) (layer "B.Cu") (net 7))
 (segment (start 243.599114 71.402284) (end 242.182321 72.819077) (width 0.2) (layer "B.Cu") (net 7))
 (segment (start 249.602 95.739306) (end 249.074206 96.2671) (width 0.2) (layer "B.Cu") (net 11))
 (segment (start 249.074206 96.2671) (end 249.074206 116.515291) (width 0.2) (layer "B.Cu") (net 11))
 (segment (start 249.602 52.347864) (end 249.602 95.739306) (width 0.2) (layer "B.Cu") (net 11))
 (segment (start 228.480127 137.10937) (end 228.480127 139.329027) (width 0.2) (layer "B.Cu") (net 11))
 (segment (start 243.524136 46.27) (end 249.602 52.347864) (width 0.2) (layer "B.Cu") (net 11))
 (segment (start 239.199705 46.27) (end 243.524136 46.27) (width 0.2) (layer "B.Cu") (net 11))
 (segment (start 249.074206 116.515291) (end 228.480127 137.10937) (width 0.2) (layer "B.Cu") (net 11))
 (segment (start 231.551887 41.66676) (end 231.26061 41.958037) (width 0.2) (layer "F.Cu") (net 9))
 (segment (start 229 38.169) (end 229.007647 38.169) (width 0.2) (layer "F.Cu") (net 9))
 (segment (start 229.007647 38.169) (end 231.551887 40.71324) (width 0.2) (layer "F.Cu") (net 9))
 (segment (start 231.26061 41.958037) (end 231.26061 56.515679) (width 0.2) (layer "F.Cu") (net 9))
 (segment (start 239.329027 64.584096) (end 239.329027 71.519873) (width 0.2) (layer "F.Cu") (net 9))
 (segment (start 231.551887 40.71324) (end 231.551887 41.66676) (width 0.2) (layer "F.Cu") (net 9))
 (segment (start 231.26061 56.515679) (end 239.329027 64.584096) (width 0.2) (layer "F.Cu") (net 9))
 (via (at 229 38.169) (size 0.6) (drill 0.3) (layers "F.Cu" "B.Cu") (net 9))
 (segment (start 219.402364 34.84) (end 222.889533 34.84) (width 0.2) (layer "B.Cu") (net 9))
 (segment (start 227.81 36.979) (end 229 38.169) (width 0.2) (layer "B.Cu") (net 9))
 (segment (start 222.889533 34.84) (end 225.028533 36.979) (width 0.2) (layer "B.Cu") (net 9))
 (segment (start 225.028533 36.979) (end 227.81 36.979) (width 0.2) (layer "B.Cu") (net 9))
 (segment (start 155.998 120.979468) (end 179.347559 144.329027) (width 0.2) (layer "B.Cu") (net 6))
 (segment (start 179.347559 144.329027) (end 180.180127 144.329027) (width 0.2) (layer "B.Cu") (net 6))
 (segment (start 158.608337 79.163437) (end 155.998 81.773774) (width 0.2) (layer "B.Cu") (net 6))
 (segment (start 158.608337 76.410195) (end 158.608337 79.163437) (width 0.2) (layer "B.Cu") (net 6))
 (segment (start 155.998 81.773774) (end 155.998 120.979468) (width 0.2) (layer "B.Cu") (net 6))
 (segment (start 234.800296 43.73) (end 191.288532 43.73) (width 0.2) (layer "B.Cu") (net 6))
 (segment (start 191.288532 43.73) (end 158.608337 76.410195) (width 0.2) (layer "B.Cu") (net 6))
 (segment (start 179.329537 140.990663) (end 186.638874 148.3) (width 0.2) (layer "B.Cu") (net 12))
 (segment (start 159.009337 79.329537) (end 156.399 81.939874) (width 0.2) (layer "B.Cu") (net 12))
 (segment (start 156.399 120.813368) (end 176.576295 140.990663) (width 0.2) (layer "B.Cu") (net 12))
 (segment (start 186.638874 148.3) (end 205 148.3) (width 0.2) (layer "B.Cu") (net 12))
 (segment (start 159.009337 76.576295) (end 159.009337 79.329537) (width 0.2) (layer "B.Cu") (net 12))
 (segment (start 190.585632 45) (end 159.009337 76.576295) (width 0.2) (layer "B.Cu") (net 12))
 (segment (start 176.576295 140.990663) (end 179.329537 140.990663) (width 0.2) (layer "B.Cu") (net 12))
 (segment (start 156.399 81.939874) (end 156.399 120.813368) (width 0.2) (layer "B.Cu") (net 12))
 (segment (start 237 45) (end 190.585632 45) (width 0.2) (layer "B.Cu") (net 12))
 (segment (start 246.1 83.126229) (end 239.923771 76.95) (width 0.2) (layer "F.Cu") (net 2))
 (segment (start 243.835341 118.872962) (end 243.472705 119.501066) (width 0.2) (layer "F.Cu") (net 2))
 (segment (start 216.873771 146.1) (end 223.05 139.923771) (width 0.2) (layer "F.Cu") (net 2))
 (segment (start 176.95 139.923771) (end 160.076229 123.05) (width 0.2) (layer "F.Cu") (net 2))
 (segment (start 243.472705 119.501066) (end 239.923771 123.05) (width 0.2) (layer "F.Cu") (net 2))
 (segment (start 223.05 60.076229) (end 239.923771 76.95) (width 0.2) (layer "F.Cu") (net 2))
 (segment (start 221.737355 60.076229) (end 215.561126 53.9) (width 0.2) (layer "F.Cu") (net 2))
 (segment (start 153.9 100) (end 153.9 116.873771) (width 0.2) (layer "F.Cu") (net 2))
 (segment (start 153.9 116.873771) (end 155.026229 118) (width 0.2) (layer "F.Cu") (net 2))
 (segment (start 153.9 100) (end 153.9 83.391697) (width 0.2) (layer "F.Cu") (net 2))
 (segment (start 183.126229 53.9) (end 200 53.9) (width 0.2) (layer "F.Cu") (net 2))
 (segment (start 200 146.1) (end 216.873771 146.1) (width 0.2) (layer "F.Cu") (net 2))
 (segment (start 156.527295 80.498934) (end 160.076229 76.95) (width 0.2) (layer "F.Cu") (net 2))
 (segment (start 176.95 60.076229) (end 160.076229 76.95) (width 0.2) (layer "F.Cu") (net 2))
 (segment (start 246.1 100) (end 246.1 116.608303) (width 0.2) (layer "F.Cu") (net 2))
 (segment (start 215.561126 53.9) (end 200 53.9) (width 0.2) (layer "F.Cu") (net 2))
 (segment (start 153.9 83.391697) (end 156.164659 81.127038) (width 0.2) (layer "F.Cu") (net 2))
 (segment (start 176.95 60.076229) (end 183.126229 53.9) (width 0.2) (layer "F.Cu") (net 2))
 (segment (start 246.1 100) (end 246.1 83.126229) (width 0.2) (layer "F.Cu") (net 2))
 (segment (start 223.05 60.076229) (end 221.737355 60.076229) (width 0.2) (layer "F.Cu") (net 2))
 (segment (start 246.1 116.608303) (end 243.835341 118.872962) (width 0.2) (layer "F.Cu") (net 2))
 (segment (start 137 118) (end 155.026229 118) (width 0.2) (layer "F.Cu") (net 2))
 (segment (start 155.026229 118) (end 160.076229 123.05) (width 0.2) (layer "F.Cu") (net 2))
 (segment (start 156.164659 81.127038) (end 156.527295 80.498934) (width 0.2) (layer "F.Cu") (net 2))
 (segment (start 223.05 139.923771) (end 239.923771 123.05) (width 0.2) (layer "F.Cu") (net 2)))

